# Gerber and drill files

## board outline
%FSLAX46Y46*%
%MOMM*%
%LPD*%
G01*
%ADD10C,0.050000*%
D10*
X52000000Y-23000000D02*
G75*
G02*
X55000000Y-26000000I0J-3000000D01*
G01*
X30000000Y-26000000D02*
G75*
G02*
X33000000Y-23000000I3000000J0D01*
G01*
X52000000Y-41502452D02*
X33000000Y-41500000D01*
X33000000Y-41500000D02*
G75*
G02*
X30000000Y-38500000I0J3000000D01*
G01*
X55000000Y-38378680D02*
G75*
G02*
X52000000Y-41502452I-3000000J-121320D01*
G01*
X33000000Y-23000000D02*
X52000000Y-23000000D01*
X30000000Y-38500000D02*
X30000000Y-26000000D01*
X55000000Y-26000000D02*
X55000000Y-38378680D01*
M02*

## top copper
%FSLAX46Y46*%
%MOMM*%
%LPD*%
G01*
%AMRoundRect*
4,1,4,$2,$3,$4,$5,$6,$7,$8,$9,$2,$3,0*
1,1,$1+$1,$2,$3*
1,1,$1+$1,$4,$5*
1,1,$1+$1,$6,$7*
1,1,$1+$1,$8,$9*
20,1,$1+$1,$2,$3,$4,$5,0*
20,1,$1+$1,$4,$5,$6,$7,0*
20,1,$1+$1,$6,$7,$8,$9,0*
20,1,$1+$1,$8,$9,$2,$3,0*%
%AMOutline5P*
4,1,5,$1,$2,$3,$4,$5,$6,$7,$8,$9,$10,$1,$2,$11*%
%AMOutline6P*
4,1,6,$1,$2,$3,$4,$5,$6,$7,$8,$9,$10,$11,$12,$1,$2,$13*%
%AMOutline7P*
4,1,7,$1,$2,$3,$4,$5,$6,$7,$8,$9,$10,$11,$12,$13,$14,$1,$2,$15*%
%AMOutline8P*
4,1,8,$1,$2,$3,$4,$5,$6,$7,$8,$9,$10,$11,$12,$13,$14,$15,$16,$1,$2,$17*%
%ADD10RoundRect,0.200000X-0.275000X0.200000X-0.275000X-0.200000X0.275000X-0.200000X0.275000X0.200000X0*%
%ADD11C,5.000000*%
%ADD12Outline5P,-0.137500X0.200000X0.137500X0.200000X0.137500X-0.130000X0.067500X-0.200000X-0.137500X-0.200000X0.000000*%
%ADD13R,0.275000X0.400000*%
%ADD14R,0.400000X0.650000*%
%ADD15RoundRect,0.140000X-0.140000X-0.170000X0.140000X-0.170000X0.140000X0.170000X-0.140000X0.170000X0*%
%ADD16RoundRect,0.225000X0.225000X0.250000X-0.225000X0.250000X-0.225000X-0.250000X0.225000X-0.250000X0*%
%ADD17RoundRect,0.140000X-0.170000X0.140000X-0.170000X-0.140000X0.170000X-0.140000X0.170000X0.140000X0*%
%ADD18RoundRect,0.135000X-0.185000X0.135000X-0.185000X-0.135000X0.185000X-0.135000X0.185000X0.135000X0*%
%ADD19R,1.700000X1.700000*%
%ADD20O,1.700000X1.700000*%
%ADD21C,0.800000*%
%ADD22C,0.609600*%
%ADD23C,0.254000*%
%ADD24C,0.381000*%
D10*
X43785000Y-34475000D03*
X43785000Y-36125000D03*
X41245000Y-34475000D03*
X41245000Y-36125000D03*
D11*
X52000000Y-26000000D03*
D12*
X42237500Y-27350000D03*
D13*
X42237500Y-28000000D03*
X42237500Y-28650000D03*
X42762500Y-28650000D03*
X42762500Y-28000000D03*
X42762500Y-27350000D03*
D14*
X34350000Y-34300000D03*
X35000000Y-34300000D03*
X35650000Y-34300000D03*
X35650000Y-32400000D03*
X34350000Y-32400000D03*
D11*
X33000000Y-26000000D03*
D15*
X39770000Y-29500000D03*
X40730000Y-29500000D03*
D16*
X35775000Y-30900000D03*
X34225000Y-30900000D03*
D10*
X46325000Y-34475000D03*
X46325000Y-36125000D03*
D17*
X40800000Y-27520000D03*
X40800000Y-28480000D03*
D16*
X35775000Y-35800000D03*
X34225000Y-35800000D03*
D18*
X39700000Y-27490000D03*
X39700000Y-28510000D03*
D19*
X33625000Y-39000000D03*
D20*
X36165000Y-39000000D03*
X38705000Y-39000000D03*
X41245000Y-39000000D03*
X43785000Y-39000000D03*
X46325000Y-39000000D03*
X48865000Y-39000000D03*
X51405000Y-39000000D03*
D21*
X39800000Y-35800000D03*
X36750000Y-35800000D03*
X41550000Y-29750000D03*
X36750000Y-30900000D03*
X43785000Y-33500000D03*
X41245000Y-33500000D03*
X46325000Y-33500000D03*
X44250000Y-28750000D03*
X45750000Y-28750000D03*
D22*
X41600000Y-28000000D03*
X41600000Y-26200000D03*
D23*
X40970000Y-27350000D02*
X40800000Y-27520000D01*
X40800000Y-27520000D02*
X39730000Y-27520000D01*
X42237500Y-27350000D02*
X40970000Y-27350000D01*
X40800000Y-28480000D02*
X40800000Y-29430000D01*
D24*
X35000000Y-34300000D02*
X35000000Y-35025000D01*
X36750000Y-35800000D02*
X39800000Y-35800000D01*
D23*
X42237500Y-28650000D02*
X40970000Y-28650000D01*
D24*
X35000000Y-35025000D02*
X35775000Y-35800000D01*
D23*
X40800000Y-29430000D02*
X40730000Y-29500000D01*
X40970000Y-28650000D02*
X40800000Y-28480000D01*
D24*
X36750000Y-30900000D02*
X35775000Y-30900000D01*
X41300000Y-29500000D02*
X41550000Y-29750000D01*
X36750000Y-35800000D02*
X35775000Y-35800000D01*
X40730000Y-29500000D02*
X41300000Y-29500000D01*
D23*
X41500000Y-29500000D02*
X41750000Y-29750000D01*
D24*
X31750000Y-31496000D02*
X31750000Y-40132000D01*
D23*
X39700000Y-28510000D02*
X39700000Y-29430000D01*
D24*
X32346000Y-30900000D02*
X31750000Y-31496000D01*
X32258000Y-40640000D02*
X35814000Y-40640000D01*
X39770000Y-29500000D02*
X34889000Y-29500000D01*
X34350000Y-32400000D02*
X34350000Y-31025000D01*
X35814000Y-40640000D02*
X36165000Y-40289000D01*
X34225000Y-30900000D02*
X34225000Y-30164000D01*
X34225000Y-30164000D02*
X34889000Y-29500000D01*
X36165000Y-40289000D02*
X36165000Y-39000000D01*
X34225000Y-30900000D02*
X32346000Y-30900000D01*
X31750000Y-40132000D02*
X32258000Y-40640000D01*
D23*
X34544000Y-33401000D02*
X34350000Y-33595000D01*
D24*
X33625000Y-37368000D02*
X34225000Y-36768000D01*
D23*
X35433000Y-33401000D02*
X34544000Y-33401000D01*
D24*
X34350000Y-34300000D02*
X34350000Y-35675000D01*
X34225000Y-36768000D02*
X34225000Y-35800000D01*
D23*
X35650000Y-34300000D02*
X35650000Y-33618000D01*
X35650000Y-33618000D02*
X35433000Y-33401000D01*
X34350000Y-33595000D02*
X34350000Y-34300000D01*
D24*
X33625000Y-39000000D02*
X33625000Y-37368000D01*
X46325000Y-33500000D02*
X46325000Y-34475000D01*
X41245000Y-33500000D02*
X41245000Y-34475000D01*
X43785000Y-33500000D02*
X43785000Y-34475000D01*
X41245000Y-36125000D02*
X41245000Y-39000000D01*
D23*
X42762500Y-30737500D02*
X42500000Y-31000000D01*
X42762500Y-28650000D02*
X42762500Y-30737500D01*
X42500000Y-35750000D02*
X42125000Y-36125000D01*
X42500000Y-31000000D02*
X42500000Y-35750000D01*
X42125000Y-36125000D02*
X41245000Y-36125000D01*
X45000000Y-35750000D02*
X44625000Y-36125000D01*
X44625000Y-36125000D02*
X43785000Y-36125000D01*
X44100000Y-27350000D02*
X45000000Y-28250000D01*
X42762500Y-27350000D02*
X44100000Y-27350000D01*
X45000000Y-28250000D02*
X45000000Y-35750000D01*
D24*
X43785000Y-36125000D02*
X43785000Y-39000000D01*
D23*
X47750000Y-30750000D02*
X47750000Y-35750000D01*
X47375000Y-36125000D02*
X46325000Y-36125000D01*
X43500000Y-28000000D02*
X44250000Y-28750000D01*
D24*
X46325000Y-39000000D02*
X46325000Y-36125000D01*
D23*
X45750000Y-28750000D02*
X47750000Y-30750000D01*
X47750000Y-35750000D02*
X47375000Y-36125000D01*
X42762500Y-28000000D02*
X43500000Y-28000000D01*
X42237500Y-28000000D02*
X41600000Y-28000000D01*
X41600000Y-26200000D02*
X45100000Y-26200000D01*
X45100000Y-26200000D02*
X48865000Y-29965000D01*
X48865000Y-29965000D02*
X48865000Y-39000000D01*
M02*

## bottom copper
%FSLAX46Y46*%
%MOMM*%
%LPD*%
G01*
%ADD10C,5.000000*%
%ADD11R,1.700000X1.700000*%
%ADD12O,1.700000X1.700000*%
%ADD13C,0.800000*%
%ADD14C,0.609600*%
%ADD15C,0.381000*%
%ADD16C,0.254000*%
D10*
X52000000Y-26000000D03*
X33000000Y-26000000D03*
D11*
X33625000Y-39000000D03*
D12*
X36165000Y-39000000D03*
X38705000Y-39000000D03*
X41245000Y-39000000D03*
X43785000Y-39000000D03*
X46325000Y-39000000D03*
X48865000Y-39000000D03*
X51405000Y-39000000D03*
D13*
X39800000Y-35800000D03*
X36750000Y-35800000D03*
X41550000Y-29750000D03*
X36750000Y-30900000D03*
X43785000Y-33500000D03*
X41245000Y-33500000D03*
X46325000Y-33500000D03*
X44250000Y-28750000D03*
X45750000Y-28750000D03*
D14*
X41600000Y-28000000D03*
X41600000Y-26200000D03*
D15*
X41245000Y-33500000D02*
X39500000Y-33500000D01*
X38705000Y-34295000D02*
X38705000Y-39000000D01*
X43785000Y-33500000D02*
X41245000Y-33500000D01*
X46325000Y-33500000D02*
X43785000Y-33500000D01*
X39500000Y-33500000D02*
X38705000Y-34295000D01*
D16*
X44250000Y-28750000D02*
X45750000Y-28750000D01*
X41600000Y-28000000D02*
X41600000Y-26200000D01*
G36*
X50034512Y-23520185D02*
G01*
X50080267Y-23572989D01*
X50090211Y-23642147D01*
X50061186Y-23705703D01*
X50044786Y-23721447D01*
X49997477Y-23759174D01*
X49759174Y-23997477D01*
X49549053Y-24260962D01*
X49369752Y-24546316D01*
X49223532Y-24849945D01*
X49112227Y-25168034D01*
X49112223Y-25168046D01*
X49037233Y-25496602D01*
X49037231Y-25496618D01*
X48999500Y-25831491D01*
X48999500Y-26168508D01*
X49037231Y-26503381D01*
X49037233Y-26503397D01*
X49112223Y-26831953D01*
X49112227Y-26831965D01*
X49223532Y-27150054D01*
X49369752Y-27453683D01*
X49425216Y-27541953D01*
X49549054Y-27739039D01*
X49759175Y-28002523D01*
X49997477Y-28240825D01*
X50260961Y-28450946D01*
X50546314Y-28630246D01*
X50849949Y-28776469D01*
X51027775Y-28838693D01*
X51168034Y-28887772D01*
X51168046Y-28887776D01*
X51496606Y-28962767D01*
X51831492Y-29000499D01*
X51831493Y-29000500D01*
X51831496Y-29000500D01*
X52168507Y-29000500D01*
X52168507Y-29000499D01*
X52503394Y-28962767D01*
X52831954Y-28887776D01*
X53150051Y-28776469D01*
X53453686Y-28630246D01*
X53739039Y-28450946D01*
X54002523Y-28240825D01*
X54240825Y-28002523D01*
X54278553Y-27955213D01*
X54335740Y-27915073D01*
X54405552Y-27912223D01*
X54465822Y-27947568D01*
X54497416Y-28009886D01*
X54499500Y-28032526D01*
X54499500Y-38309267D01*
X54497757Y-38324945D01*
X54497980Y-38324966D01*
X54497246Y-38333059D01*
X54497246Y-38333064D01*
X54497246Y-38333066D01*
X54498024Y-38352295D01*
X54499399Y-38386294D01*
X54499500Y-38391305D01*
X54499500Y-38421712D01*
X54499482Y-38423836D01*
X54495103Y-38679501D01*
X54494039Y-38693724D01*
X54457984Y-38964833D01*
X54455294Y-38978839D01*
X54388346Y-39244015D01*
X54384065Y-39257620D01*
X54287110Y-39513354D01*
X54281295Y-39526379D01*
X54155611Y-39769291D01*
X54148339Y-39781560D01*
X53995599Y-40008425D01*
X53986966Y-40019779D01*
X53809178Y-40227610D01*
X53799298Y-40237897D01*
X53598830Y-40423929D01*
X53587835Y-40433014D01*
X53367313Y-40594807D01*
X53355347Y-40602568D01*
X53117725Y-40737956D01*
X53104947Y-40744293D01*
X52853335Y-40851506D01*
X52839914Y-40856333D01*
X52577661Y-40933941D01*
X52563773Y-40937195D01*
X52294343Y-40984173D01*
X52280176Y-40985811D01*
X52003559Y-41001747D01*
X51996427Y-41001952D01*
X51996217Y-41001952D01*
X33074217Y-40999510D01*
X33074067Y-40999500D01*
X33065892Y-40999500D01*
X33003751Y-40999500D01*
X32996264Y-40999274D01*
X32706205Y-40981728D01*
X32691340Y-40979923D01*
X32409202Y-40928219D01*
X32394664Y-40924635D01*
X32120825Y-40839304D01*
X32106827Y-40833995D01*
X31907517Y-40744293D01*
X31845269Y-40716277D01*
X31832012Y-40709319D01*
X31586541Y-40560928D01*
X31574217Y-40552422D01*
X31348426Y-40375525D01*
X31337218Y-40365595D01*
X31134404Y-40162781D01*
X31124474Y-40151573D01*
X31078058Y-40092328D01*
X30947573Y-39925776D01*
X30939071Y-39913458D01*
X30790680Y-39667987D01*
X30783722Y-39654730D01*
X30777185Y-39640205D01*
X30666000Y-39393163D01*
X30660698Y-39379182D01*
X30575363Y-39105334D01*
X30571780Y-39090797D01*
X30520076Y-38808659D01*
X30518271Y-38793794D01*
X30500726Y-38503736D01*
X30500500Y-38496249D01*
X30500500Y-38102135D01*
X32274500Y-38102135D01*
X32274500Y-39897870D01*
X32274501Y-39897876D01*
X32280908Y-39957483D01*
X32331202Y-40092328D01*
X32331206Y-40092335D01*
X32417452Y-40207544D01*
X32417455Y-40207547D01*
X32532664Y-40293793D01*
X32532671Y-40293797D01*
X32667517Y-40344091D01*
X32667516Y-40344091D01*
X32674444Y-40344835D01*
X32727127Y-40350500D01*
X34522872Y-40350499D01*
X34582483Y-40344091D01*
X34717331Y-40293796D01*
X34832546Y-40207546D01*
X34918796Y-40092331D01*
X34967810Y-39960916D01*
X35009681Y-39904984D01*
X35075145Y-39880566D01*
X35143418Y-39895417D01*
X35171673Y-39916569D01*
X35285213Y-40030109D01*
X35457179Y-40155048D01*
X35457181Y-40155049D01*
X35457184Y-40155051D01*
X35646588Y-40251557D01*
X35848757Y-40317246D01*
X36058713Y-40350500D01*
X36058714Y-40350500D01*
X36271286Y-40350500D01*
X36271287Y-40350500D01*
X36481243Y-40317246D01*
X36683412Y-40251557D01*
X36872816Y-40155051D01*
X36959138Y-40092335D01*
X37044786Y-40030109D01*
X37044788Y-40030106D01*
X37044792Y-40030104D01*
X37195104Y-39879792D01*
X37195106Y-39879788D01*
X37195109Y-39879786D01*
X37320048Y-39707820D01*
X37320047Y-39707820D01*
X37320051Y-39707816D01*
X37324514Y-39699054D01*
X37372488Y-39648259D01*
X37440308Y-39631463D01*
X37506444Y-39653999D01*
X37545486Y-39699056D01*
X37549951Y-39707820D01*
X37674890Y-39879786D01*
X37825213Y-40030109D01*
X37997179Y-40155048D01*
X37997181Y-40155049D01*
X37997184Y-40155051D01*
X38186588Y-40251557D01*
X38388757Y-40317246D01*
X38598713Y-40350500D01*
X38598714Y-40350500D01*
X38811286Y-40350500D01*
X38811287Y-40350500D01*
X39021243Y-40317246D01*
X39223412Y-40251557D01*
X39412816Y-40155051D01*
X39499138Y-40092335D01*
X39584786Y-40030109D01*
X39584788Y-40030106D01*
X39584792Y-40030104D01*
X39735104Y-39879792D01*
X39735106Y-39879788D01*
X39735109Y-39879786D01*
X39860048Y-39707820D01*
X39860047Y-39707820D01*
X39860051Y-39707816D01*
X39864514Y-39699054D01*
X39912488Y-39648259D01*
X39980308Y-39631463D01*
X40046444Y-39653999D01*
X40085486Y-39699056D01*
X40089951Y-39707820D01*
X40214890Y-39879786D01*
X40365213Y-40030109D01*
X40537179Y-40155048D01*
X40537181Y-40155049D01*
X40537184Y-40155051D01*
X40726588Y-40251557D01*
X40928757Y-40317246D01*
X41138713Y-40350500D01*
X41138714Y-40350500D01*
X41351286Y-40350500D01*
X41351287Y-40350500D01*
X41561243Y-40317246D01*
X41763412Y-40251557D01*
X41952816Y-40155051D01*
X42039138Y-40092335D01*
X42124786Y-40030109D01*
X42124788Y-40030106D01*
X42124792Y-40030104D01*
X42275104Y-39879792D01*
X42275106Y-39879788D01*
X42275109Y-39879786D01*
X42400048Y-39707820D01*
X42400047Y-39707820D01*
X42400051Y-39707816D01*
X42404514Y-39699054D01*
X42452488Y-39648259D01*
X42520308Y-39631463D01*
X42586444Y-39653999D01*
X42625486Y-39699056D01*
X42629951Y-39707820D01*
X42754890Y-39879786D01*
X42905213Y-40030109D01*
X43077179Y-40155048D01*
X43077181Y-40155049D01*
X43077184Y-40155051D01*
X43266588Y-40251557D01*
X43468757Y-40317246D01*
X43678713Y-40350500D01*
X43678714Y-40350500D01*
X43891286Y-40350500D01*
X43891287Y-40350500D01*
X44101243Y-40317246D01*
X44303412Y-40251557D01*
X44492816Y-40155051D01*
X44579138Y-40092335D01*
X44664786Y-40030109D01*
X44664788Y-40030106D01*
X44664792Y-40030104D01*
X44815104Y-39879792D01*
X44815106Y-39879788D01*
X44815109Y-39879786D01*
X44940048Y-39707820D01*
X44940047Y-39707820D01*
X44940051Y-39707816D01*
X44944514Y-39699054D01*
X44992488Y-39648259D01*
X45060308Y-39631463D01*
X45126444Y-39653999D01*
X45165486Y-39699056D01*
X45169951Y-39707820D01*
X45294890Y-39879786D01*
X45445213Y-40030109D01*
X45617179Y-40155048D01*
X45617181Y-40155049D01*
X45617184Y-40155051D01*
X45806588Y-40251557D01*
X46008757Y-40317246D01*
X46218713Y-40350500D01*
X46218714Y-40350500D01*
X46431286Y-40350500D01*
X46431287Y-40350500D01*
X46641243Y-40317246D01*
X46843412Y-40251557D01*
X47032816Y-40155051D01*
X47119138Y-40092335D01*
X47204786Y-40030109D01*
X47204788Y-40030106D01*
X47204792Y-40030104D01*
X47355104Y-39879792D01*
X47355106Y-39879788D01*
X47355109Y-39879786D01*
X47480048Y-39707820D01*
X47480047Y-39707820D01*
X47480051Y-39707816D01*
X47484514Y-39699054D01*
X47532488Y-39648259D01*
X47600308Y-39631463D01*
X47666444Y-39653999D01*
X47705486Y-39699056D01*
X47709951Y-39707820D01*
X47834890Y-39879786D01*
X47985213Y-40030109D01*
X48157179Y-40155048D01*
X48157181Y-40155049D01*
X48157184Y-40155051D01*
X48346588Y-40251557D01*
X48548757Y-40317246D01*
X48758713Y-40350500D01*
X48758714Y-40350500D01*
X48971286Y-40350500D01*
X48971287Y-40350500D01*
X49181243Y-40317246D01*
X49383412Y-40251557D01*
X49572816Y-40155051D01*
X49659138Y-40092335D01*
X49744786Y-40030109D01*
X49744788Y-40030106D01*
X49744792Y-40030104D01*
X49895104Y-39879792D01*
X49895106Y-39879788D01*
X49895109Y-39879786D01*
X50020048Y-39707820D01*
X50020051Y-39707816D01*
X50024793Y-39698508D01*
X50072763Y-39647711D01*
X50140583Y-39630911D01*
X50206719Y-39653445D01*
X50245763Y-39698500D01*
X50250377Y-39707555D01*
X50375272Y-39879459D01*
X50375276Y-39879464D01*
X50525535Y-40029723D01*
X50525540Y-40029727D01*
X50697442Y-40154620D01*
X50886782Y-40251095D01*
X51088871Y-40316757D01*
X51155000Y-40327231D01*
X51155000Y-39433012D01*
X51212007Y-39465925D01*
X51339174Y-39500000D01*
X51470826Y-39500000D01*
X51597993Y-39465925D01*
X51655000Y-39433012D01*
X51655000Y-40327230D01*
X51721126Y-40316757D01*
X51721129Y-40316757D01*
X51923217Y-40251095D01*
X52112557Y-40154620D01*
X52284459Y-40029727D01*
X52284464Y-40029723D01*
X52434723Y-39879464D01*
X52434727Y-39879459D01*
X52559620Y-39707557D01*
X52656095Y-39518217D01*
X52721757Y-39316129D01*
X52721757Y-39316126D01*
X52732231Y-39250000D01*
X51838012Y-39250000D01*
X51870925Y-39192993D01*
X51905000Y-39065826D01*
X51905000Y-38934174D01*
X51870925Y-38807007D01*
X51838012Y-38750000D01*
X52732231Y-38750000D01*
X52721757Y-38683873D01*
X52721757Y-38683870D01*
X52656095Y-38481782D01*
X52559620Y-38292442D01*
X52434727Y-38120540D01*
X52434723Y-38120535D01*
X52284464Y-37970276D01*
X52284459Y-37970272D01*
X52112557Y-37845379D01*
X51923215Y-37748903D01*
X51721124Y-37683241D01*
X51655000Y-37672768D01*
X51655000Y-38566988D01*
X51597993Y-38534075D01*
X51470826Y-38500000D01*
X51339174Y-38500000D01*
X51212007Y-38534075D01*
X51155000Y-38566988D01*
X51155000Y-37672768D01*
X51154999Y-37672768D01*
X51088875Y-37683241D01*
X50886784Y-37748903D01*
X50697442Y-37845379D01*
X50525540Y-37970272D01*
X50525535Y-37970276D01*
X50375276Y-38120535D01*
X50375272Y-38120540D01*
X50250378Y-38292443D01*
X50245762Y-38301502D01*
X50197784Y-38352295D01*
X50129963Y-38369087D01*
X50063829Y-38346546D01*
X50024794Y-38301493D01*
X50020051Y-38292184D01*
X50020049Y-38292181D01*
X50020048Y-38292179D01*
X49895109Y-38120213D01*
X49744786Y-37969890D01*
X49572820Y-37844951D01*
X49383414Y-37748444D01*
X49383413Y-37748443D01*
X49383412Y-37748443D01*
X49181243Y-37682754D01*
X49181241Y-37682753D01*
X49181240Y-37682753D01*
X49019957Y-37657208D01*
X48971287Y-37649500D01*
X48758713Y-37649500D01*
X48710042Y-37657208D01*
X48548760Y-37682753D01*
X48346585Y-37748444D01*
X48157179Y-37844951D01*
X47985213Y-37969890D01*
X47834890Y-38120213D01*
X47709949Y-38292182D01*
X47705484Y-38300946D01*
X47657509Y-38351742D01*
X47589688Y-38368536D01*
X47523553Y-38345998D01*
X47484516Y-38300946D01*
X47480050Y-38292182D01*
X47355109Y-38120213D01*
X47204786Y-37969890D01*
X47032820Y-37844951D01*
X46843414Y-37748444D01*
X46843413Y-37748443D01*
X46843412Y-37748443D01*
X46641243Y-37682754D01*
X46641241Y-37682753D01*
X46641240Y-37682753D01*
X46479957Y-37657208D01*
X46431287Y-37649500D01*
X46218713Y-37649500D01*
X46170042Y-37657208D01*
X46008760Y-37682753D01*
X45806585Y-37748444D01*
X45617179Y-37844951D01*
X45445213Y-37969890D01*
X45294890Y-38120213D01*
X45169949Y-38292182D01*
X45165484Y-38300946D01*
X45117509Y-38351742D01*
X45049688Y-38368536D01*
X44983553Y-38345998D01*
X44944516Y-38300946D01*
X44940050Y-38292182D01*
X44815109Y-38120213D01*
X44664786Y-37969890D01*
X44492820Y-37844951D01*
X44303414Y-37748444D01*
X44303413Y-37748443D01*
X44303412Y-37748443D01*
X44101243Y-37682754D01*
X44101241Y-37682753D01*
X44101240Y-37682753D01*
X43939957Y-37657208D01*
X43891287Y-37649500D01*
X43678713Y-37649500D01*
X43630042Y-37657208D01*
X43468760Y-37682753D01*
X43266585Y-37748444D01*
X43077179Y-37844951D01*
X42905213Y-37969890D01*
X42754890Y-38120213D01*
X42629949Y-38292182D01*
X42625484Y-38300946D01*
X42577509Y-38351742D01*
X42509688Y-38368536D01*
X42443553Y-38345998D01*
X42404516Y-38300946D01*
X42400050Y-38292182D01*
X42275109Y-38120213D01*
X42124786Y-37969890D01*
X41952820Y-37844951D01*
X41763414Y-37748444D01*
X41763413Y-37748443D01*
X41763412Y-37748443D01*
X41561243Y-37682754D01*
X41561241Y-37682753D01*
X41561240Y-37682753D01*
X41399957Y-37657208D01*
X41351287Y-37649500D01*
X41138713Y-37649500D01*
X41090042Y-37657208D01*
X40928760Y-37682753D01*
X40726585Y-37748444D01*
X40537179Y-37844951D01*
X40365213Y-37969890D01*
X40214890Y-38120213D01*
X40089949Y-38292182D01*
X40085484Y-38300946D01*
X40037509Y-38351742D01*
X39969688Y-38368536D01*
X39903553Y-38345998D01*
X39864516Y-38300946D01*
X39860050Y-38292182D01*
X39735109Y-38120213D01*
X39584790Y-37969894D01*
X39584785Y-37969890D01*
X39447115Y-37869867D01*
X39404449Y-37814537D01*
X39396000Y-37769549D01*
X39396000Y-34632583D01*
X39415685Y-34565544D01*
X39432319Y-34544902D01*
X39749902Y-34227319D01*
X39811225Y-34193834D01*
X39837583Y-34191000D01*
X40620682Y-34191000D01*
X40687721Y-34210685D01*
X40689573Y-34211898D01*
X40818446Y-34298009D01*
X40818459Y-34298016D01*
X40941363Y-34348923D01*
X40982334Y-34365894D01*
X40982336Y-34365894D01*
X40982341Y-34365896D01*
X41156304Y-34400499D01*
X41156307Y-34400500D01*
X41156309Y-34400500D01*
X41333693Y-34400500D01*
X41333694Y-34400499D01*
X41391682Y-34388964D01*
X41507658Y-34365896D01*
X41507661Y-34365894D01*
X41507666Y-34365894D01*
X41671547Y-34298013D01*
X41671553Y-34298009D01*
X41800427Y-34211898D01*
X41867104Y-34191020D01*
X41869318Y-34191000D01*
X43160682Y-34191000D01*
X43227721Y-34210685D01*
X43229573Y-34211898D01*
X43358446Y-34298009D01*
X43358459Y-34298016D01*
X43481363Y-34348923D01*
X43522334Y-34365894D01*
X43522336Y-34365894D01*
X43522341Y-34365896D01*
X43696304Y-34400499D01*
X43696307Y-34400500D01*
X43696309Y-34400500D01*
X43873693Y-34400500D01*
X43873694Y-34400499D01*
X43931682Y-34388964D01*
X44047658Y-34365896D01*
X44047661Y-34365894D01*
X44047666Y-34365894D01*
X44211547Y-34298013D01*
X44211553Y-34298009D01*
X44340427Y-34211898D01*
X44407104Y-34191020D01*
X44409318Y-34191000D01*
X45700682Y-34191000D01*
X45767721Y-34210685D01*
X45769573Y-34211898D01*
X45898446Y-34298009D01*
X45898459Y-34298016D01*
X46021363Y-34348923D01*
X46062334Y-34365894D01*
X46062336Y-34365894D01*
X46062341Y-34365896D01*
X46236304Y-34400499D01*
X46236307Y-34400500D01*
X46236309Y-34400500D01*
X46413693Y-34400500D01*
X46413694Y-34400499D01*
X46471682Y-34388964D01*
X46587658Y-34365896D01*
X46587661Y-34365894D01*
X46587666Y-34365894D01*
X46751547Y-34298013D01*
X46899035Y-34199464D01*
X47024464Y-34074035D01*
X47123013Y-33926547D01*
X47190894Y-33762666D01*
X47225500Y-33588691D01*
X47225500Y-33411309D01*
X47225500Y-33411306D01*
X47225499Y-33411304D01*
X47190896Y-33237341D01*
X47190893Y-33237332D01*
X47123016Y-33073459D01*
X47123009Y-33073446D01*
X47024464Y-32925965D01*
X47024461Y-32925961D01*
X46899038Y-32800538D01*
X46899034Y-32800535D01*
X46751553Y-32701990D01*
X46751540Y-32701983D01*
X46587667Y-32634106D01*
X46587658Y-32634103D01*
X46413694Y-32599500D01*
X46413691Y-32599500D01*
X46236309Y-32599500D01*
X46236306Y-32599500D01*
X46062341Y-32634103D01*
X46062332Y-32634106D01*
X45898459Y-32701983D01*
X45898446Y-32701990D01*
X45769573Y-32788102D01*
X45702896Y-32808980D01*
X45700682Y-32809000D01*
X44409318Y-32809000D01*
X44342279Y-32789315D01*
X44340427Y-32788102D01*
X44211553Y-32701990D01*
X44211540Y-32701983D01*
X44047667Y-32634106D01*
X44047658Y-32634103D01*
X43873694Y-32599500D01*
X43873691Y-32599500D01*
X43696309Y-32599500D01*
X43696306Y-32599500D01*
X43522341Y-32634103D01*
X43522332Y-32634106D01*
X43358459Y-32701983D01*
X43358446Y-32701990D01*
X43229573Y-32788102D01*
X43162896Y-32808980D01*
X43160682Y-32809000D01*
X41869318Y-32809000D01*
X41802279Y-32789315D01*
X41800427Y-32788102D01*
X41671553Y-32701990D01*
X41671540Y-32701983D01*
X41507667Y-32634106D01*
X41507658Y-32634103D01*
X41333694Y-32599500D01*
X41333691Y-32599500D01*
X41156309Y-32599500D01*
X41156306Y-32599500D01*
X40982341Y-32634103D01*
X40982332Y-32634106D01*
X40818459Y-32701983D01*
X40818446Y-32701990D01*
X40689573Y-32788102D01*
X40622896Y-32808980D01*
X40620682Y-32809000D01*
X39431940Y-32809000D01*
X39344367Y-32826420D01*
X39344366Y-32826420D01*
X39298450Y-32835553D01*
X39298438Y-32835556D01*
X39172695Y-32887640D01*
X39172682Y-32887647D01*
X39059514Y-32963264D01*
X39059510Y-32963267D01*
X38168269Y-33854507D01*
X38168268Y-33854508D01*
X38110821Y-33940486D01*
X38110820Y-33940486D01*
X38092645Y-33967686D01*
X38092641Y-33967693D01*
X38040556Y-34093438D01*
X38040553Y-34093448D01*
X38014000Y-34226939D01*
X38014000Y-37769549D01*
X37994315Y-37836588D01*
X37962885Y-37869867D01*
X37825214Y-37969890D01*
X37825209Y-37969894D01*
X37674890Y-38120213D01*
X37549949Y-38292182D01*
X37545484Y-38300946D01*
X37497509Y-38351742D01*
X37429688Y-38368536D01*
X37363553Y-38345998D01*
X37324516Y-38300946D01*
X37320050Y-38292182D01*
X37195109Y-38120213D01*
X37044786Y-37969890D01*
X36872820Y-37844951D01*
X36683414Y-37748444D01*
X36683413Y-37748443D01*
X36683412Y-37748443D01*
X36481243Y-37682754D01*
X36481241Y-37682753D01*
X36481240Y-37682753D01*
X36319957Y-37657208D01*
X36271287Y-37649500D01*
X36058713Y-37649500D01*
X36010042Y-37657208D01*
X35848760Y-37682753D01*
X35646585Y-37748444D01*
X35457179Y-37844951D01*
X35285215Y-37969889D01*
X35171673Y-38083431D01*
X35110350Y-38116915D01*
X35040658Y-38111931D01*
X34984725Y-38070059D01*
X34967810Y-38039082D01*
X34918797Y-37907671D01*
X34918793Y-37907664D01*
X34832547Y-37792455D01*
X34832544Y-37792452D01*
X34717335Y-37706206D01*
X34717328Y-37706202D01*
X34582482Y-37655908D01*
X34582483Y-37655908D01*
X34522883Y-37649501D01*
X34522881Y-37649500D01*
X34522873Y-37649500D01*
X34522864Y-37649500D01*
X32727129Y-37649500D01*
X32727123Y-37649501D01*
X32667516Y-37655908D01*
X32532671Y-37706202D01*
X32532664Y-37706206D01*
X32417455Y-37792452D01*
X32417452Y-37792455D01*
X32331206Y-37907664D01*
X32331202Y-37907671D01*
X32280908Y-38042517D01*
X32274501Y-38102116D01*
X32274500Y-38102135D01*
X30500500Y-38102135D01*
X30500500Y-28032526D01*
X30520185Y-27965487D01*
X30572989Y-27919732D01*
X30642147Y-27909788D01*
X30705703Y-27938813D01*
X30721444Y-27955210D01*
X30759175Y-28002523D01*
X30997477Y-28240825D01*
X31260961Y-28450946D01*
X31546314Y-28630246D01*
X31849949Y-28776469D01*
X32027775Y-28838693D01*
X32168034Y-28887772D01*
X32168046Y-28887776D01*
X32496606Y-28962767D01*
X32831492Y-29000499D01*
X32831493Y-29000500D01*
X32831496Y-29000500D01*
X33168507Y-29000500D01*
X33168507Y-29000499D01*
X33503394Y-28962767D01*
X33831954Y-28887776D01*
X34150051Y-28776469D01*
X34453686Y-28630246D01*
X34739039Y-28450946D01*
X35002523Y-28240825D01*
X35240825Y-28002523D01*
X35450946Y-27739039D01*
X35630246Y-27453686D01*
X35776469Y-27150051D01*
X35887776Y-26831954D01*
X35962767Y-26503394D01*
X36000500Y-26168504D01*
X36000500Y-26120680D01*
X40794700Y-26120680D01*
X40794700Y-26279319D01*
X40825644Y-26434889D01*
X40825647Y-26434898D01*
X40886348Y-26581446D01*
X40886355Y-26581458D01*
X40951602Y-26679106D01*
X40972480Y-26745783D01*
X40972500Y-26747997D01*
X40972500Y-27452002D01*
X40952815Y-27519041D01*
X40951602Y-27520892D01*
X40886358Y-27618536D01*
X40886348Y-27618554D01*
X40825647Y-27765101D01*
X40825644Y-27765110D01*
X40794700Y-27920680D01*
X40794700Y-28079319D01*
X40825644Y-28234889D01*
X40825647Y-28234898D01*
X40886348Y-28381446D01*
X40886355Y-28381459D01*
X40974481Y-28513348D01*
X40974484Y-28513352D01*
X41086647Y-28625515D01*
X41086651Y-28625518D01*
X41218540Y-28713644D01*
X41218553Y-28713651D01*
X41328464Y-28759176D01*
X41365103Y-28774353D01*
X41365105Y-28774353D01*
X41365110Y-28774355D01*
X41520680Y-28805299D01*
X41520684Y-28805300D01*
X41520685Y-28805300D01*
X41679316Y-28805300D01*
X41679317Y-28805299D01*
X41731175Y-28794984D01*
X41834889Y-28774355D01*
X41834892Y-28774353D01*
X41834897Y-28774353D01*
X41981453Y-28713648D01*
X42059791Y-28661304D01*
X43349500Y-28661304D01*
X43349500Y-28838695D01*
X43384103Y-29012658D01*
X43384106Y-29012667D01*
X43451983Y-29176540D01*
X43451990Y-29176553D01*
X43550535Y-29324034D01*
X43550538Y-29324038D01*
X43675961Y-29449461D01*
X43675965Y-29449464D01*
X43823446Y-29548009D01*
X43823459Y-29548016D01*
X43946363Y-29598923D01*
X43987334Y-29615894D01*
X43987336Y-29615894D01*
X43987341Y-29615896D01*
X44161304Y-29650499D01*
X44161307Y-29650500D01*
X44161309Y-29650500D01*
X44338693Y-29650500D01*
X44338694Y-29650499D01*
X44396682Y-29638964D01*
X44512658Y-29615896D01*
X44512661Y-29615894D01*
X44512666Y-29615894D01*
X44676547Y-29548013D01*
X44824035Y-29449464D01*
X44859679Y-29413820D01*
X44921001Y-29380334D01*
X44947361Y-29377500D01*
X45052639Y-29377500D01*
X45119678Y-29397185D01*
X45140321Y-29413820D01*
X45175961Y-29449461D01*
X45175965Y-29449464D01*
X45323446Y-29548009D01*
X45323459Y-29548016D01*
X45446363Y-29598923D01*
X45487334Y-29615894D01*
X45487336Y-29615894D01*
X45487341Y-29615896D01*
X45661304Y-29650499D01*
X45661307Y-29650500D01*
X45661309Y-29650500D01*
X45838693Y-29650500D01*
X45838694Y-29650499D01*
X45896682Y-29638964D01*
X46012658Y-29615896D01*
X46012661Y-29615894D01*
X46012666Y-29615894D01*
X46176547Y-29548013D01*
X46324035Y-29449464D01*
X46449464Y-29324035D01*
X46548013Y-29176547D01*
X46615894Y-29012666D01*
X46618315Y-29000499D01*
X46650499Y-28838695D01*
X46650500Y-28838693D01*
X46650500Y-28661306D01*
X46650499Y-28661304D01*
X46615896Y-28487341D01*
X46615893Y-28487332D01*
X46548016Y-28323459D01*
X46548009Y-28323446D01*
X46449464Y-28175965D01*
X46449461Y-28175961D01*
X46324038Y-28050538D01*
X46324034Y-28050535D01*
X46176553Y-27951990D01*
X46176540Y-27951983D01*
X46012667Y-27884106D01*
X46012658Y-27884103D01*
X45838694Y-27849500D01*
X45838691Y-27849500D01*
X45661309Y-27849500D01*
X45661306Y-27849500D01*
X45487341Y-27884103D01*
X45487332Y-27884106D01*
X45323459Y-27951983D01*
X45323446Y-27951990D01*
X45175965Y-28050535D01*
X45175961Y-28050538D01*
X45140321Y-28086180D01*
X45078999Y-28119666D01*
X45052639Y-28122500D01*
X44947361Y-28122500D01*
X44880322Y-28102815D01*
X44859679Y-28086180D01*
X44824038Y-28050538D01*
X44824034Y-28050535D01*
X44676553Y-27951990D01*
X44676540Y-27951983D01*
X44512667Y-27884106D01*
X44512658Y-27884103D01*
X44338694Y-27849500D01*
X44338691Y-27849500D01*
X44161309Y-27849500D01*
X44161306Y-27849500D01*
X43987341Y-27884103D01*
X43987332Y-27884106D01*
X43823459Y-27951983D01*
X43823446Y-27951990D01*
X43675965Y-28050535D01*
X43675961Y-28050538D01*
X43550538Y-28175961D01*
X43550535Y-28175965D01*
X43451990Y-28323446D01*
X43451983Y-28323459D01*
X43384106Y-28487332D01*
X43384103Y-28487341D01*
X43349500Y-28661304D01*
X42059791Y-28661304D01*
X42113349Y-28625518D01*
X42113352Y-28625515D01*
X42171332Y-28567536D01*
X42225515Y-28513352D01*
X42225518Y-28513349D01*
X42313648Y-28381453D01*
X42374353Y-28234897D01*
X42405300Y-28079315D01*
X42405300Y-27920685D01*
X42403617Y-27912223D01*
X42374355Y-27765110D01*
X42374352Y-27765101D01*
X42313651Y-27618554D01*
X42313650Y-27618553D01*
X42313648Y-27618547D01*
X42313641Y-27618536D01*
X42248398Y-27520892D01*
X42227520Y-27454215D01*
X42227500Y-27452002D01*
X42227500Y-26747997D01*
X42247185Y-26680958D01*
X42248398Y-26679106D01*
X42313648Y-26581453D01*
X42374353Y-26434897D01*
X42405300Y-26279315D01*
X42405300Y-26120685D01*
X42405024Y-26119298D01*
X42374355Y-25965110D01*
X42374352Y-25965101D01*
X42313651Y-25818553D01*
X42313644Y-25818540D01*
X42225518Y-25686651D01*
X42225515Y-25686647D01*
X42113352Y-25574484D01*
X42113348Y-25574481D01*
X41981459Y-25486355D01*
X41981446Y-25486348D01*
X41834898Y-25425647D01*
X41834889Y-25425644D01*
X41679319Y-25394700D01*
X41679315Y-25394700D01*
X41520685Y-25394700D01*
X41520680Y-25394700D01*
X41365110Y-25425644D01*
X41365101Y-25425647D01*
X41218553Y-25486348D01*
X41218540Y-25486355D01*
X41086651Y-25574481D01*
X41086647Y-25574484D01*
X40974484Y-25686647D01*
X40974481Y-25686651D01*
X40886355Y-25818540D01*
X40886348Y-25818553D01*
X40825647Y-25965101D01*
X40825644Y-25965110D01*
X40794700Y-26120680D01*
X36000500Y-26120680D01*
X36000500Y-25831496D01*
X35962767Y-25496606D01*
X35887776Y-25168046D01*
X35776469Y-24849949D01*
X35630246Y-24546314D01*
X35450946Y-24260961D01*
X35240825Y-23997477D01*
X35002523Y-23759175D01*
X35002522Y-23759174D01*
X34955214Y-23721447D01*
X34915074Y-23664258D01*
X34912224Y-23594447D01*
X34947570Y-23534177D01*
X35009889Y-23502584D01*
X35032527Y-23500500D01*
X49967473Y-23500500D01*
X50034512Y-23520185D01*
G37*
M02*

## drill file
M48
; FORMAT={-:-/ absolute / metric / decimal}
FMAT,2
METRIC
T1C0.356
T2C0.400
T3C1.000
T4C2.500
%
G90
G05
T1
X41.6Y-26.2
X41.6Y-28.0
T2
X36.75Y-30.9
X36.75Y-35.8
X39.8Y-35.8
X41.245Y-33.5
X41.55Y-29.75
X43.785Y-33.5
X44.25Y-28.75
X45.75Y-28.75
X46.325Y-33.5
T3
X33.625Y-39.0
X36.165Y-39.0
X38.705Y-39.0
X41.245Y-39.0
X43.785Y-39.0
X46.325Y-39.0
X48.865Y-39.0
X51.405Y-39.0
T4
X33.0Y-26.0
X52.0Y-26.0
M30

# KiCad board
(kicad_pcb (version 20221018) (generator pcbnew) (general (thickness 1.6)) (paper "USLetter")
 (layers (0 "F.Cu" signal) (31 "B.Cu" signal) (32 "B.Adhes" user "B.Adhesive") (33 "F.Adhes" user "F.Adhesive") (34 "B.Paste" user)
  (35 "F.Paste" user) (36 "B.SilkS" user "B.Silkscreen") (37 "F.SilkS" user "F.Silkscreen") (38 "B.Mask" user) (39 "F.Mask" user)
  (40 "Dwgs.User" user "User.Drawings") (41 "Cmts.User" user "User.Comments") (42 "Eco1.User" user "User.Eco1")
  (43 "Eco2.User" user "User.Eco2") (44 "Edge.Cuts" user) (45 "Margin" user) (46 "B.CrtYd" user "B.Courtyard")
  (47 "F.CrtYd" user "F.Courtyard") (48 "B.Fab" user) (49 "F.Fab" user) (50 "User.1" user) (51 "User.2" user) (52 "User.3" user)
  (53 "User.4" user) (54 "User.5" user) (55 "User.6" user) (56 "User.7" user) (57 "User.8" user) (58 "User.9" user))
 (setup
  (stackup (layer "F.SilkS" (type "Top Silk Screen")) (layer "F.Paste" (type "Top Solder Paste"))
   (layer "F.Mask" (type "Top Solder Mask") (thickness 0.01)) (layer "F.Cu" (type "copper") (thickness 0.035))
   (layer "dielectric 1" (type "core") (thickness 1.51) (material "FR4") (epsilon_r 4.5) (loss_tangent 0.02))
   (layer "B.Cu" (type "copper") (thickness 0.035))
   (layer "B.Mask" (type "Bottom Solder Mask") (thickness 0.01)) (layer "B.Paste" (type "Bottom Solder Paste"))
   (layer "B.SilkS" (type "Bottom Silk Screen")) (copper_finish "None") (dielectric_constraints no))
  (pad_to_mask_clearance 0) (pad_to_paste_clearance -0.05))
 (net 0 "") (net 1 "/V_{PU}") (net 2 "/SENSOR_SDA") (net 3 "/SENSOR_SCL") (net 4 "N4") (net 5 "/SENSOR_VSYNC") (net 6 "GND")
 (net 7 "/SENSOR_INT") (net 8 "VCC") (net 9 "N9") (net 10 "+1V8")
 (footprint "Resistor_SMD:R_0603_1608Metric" (layer "F.Cu") (at 43.785 35.3 -90)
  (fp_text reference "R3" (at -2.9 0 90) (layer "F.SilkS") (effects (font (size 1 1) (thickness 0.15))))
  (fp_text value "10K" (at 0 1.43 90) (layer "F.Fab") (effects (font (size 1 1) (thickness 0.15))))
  (pad "1" smd roundrect (at -0.825 0 270) (size 0.8 0.95) (layers "F.Cu" "F.Paste" "F.Mask") (roundrect_rratio 0.25) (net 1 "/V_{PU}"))
  (pad "2" smd roundrect (at 0.825 0 270) (size 0.8 0.95) (layers "F.Cu" "F.Paste" "F.Mask") (roundrect_rratio 0.25) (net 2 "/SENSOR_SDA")))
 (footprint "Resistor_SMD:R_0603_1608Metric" (layer "F.Cu") (at 41.245 35.3 -90)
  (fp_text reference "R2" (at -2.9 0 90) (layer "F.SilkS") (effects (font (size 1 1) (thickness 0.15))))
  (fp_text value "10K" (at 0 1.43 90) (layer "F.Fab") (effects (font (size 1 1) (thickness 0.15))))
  (pad "1" smd roundrect (at -0.825 0 270) (size 0.8 0.95) (layers "F.Cu" "F.Paste" "F.Mask") (roundrect_rratio 0.25) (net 1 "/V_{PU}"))
  (pad "2" smd roundrect (at 0.825 0 270) (size 0.8 0.95) (layers "F.Cu" "F.Paste" "F.Mask") (roundrect_rratio 0.25) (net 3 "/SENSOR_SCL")))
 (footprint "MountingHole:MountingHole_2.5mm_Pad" (layer "F.Cu") (at 52 26)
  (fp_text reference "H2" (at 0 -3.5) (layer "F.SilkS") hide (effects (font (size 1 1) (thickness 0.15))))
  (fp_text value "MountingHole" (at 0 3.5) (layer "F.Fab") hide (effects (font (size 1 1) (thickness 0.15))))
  (pad "1" thru_hole circle (at 0 0) (size 5 5) (drill 2.5) (layers "*.Cu" "*.Mask")))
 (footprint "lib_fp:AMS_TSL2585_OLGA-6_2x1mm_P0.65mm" (layer "F.Cu") (at 42.5 28) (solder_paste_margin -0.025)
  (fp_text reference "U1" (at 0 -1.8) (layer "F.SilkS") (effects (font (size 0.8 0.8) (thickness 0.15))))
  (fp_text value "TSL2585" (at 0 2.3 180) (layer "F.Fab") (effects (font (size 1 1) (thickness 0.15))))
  (pad "1" smd roundrect (at -0.2625 -0.65) (size 0.275 0.4) (layers "F.Cu" "F.Paste" "F.Mask") (roundrect_rratio 0)
   (chamfer_ratio 0.254545) (chamfer bottom_right) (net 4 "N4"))
  (pad "2" smd rect (at -0.2625 0) (size 0.275 0.4) (layers "F.Cu" "F.Paste" "F.Mask") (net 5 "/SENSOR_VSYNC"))
  (pad "3" smd rect (at -0.2625 0.65) (size 0.275 0.4) (layers "F.Cu" "F.Paste" "F.Mask") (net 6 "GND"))
  (pad "4" smd rect (at 0.2625 0.65) (size 0.275 0.4) (layers "F.Cu" "F.Paste" "F.Mask") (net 3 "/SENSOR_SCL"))
  (pad "5" smd rect (at 0.2625 0) (size 0.275 0.4) (layers "F.Cu" "F.Paste" "F.Mask") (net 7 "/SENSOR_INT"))
  (pad "6" smd rect (at 0.2625 -0.65) (size 0.275 0.4) (layers "F.Cu" "F.Paste" "F.Mask") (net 2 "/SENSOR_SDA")))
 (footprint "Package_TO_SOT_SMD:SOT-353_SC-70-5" (layer "F.Cu") (at 35 33.35 90)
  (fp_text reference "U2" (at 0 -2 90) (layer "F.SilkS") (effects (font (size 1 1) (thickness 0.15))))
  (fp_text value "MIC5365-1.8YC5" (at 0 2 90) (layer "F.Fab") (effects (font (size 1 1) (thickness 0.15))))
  (pad "1" smd rect (at -0.95 -0.65 90) (size 0.65 0.4) (layers "F.Cu" "F.Paste" "F.Mask") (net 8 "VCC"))
  (pad "2" smd rect (at -0.95 0 90) (size 0.65 0.4) (layers "F.Cu" "F.Paste" "F.Mask") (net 6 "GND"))
  (pad "3" smd rect (at -0.95 0.65 90) (size 0.65 0.4) (layers "F.Cu" "F.Paste" "F.Mask") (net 8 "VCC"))
  (pad "4" smd rect (at 0.95 0.65 90) (size 0.65 0.4) (layers "F.Cu" "F.Paste" "F.Mask") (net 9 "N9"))
  (pad "5" smd rect (at 0.95 -0.65 90) (size 0.65 0.4) (layers "F.Cu" "F.Paste" "F.Mask") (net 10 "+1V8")))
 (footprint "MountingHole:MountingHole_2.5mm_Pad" (layer "F.Cu") (at 33 26)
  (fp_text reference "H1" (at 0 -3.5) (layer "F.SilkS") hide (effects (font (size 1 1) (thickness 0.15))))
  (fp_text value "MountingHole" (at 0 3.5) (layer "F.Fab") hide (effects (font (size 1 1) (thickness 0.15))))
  (pad "1" thru_hole circle (at 0 0) (size 5 5) (drill 2.5) (layers "*.Cu" "*.Mask")))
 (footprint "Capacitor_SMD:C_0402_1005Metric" (layer "F.Cu") (at 40.25 29.5)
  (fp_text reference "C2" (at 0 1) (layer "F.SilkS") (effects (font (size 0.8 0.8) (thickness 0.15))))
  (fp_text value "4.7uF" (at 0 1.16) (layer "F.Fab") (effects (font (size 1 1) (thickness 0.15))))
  (pad "1" smd roundrect (at -0.48 0) (size 0.56 0.62) (layers "F.Cu" "F.Paste" "F.Mask") (roundrect_rratio 0.25) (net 10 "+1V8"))
  (pad "2" smd roundrect (at 0.48 0) (size 0.56 0.62) (layers "F.Cu" "F.Paste" "F.Mask") (roundrect_rratio 0.25) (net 6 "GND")))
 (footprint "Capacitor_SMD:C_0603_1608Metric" (layer "F.Cu") (at 35 30.9 180)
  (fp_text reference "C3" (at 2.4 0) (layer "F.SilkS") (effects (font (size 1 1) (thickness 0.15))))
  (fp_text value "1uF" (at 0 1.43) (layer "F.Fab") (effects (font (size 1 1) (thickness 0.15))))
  (pad "1" smd roundrect (at -0.775 0 180) (size 0.9 0.95) (layers "F.Cu" "F.Paste" "F.Mask") (roundrect_rratio 0.25) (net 6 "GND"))
  (pad "2" smd roundrect (at 0.775 0 180) (size 0.9 0.95) (layers "F.Cu" "F.Paste" "F.Mask") (roundrect_rratio 0.25) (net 10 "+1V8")))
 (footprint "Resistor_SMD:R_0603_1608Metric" (layer "F.Cu") (at 46.325 35.3 -90)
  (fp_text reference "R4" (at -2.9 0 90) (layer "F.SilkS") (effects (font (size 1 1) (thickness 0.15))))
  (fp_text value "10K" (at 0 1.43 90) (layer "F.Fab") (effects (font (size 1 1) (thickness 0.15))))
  (pad "1" smd roundrect (at -0.825 0 270) (size 0.8 0.95) (layers "F.Cu" "F.Paste" "F.Mask") (roundrect_rratio 0.25) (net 1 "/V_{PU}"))
  (pad "2" smd roundrect (at 0.825 0 270) (size 0.8 0.95) (layers "F.Cu" "F.Paste" "F.Mask") (roundrect_rratio 0.25) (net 7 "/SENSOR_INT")))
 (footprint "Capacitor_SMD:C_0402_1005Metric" (layer "F.Cu") (at 40.8 28 -90)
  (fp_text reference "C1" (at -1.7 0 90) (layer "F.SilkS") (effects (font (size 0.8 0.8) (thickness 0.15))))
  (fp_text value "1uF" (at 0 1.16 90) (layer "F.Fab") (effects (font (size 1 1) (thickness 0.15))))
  (pad "1" smd roundrect (at -0.48 0 270) (size 0.56 0.62) (layers "F.Cu" "F.Paste" "F.Mask") (roundrect_rratio 0.25) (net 4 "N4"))
  (pad "2" smd roundrect (at 0.48 0 270) (size 0.56 0.62) (layers "F.Cu" "F.Paste" "F.Mask") (roundrect_rratio 0.25) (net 6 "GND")))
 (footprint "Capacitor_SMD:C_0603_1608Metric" (layer "F.Cu") (at 35 35.8 180)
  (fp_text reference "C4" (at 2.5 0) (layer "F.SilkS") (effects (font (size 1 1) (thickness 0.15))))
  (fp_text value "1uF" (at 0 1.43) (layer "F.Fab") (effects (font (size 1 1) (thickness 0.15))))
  (pad "1" smd roundrect (at -0.775 0 180) (size 0.9 0.95) (layers "F.Cu" "F.Paste" "F.Mask") (roundrect_rratio 0.25) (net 6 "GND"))
  (pad "2" smd roundrect (at 0.775 0 180) (size 0.9 0.95) (layers "F.Cu" "F.Paste" "F.Mask") (roundrect_rratio 0.25) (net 8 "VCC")))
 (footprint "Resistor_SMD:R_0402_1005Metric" (layer "F.Cu") (at 39.7 28 -90)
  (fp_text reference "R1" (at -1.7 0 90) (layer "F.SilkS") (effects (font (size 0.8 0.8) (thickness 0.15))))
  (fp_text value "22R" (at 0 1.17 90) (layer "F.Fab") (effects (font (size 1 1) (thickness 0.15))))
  (pad "1" smd roundrect (at -0.51 0 270) (size 0.54 0.64) (layers "F.Cu" "F.Paste" "F.Mask") (roundrect_rratio 0.25) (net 4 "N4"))
  (pad "2" smd roundrect (at 0.51 0 270) (size 0.54 0.64) (layers "F.Cu" "F.Paste" "F.Mask") (roundrect_rratio 0.25) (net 10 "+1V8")))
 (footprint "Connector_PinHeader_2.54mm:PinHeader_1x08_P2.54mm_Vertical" (layer "B.Cu") (at 33.625 39 -90)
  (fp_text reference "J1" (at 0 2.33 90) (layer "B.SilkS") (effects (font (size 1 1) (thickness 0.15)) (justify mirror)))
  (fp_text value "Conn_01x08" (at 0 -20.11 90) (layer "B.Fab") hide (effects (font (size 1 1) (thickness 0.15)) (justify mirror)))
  (pad "1" thru_hole rect (at 0 0 270) (size 1.7 1.7) (drill 1) (layers "*.Cu" "*.Mask") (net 8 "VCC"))
  (pad "2" thru_hole oval (at 0 -2.54 270) (size 1.7 1.7) (drill 1) (layers "*.Cu" "*.Mask") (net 10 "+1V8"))
  (pad "3" thru_hole oval (at 0 -5.08 270) (size 1.7 1.7) (drill 1) (layers "*.Cu" "*.Mask") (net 1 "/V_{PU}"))
  (pad "4" thru_hole oval (at 0 -7.62 270) (size 1.7 1.7) (drill 1) (layers "*.Cu" "*.Mask") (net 3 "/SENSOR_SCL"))
  (pad "5" thru_hole oval (at 0 -10.16 270) (size 1.7 1.7) (drill 1) (layers "*.Cu" "*.Mask") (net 2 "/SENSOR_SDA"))
  (pad "6" thru_hole oval (at 0 -12.7 270) (size 1.7 1.7) (drill 1) (layers "*.Cu" "*.Mask") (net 7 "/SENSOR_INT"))
  (pad "7" thru_hole oval (at 0 -15.24 270) (size 1.7 1.7) (drill 1) (layers "*.Cu" "*.Mask") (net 5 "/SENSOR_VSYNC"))
  (pad "8" thru_hole oval (at 0 -17.78 270) (size 1.7 1.7) (drill 1) (layers "*.Cu" "*.Mask") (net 6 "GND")))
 (gr_arc (start 52 23) (mid 54.12132 23.87868) (end 55 26) (stroke (width 0.05) (type default)) (layer "Edge.Cuts"))
 (gr_arc (start 30 26) (mid 30.87868 23.87868) (end 33 23) (stroke (width 0.05) (type default)) (layer "Edge.Cuts"))
 (gr_line (start 52 41.502452) (end 33 41.5) (stroke (width 0.05) (type default)) (layer "Edge.Cuts"))
 (gr_arc (start 33 41.5) (mid 30.87868 40.62132) (end 30 38.5) (stroke (width 0.05) (type default)) (layer "Edge.Cuts"))
 (gr_arc (start 55 38.37868) (mid 54.165523 40.579719) (end 52 41.502452) (stroke (width 0.05) (type default)) (layer "Edge.Cuts"))
 (gr_line (start 33 23) (end 52 23) (stroke (width 0.05) (type default)) (layer "Edge.Cuts"))
 (gr_line (start 30 38.5) (end 30 26) (stroke (width 0.05) (type default)) (layer "Edge.Cuts"))
 (gr_line (start 55 26) (end 55 38.37868) (stroke (width 0.05) (type default)) (layer "Edge.Cuts"))
 (segment (start 40.97 27.35) (end 40.8 27.52) (width 0.254) (layer "F.Cu") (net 4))
 (segment (start 40.8 27.52) (end 39.73 27.52) (width 0.254) (layer "F.Cu") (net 4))
 (segment (start 42.2375 27.35) (end 40.97 27.35) (width 0.254) (layer "F.Cu") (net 4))
 (segment (start 40.8 28.48) (end 40.8 29.43) (width 0.254) (layer "F.Cu") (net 6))
 (segment (start 35 34.3) (end 35 35.025) (width 0.381) (layer "F.Cu") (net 6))
 (segment (start 36.75 35.8) (end 39.8 35.8) (width 0.381) (layer "F.Cu") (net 6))
 (segment (start 42.2375 28.65) (end 40.97 28.65) (width 0.254) (layer "F.Cu") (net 6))
 (segment (start 35 35.025) (end 35.775 35.8) (width 0.381) (layer "F.Cu") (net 6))
 (segment (start 40.8 29.43) (end 40.73 29.5) (width 0.254) (layer "F.Cu") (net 6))
 (segment (start 40.97 28.65) (end 40.8 28.48) (width 0.254) (layer "F.Cu") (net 6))
 (segment (start 36.75 30.9) (end 35.775 30.9) (width 0.381) (layer "F.Cu") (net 6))
 (segment (start 41.3 29.5) (end 41.55 29.75) (width 0.381) (layer "F.Cu") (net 6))
 (segment (start 36.75 35.8) (end 35.775 35.8) (width 0.381) (layer "F.Cu") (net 6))
 (segment (start 40.73 29.5) (end 41.3 29.5) (width 0.381) (layer "F.Cu") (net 6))
 (segment (start 41.5 29.5) (end 41.75 29.75) (width 0.254) (layer "F.Cu") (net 6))
 (via (at 39.8 35.8) (size 0.8) (drill 0.4) (layers "F.Cu" "B.Cu") (free) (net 6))
 (via (at 36.75 35.8) (size 0.8) (drill 0.4) (layers "F.Cu" "B.Cu") (free) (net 6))
 (via (at 41.55 29.75) (size 0.8) (drill 0.4) (layers "F.Cu" "B.Cu") (free) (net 6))
 (via (at 36.75 30.9) (size 0.8) (drill 0.4) (layers "F.Cu" "B.Cu") (free) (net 6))
 (segment (start 31.75 31.496) (end 31.75 40.132) (width 0.381) (layer "F.Cu") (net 10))
 (segment (start 39.7 28.51) (end 39.7 29.43) (width 0.254) (layer "F.Cu") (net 10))
 (segment (start 32.346 30.9) (end 31.75 31.496) (width 0.381) (layer "F.Cu") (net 10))
 (segment (start 32.258 40.64) (end 35.814 40.64) (width 0.381) (layer "F.Cu") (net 10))
 (segment (start 39.77 29.5) (end 34.889 29.5) (width 0.381) (layer "F.Cu") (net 10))
 (segment (start 34.35 32.4) (end 34.35 31.025) (width 0.381) (layer "F.Cu") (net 10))
 (segment (start 35.814 40.64) (end 36.165 40.289) (width 0.381) (layer "F.Cu") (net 10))
 (segment (start 34.225 30.9) (end 34.225 30.164) (width 0.381) (layer "F.Cu") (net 10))
 (segment (start 34.225 30.164) (end 34.889 29.5) (width 0.381) (layer "F.Cu") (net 10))
 (segment (start 36.165 40.289) (end 36.165 39) (width 0.381) (layer "F.Cu") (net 10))
 (segment (start 34.225 30.9) (end 32.346 30.9) (width 0.381) (layer "F.Cu") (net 10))
 (segment (start 31.75 40.132) (end 32.258 40.64) (width 0.381) (layer "F.Cu") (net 10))
 (segment (start 34.544 33.401) (end 34.35 33.595) (width 0.254) (layer "F.Cu") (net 8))
 (segment (start 33.625 37.368) (end 34.225 36.768) (width 0.381) (layer "F.Cu") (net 8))
 (segment (start 35.433 33.401) (end 34.544 33.401) (width 0.254) (layer "F.Cu") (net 8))
 (segment (start 34.35 34.3) (end 34.35 35.675) (width 0.381) (layer "F.Cu") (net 8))
 (segment (start 34.225 36.768) (end 34.225 35.8) (width 0.381) (layer "F.Cu") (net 8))
 (segment (start 35.65 34.3) (end 35.65 33.618) (width 0.254) (layer "F.Cu") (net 8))
 (segment (start 35.65 33.618) (end 35.433 33.401) (width 0.254) (layer "F.Cu") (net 8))
 (segment (start 34.35 33.595) (end 34.35 34.3) (width 0.254) (layer "F.Cu") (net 8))
 (segment (start 33.625 39) (end 33.625 37.368) (width 0.381) (layer "F.Cu") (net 8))
 (segment (start 46.325 33.5) (end 46.325 34.475) (width 0.381) (layer "F.Cu") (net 1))
 (segment (start 41.245 33.5) (end 41.245 34.475) (width 0.381) (layer "F.Cu") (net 1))
 (segment (start 43.785 33.5) (end 43.785 34.475) (width 0.381) (layer "F.Cu") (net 1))
 (via (at 43.785 33.5) (size 0.8) (drill 0.4) (layers "F.Cu" "B.Cu") (free) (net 1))
 (via (at 41.245 33.5) (size 0.8) (drill 0.4) (layers "F.Cu" "B.Cu") (free) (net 1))
 (via (at 46.325 33.5) (size 0.8) (drill 0.4) (layers "F.Cu" "B.Cu") (free) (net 1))
 (segment (start 41.245 33.5) (end 39.5 33.5) (width 0.381) (layer "B.Cu") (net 1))
 (segment (start 38.705 34.295) (end 38.705 39) (width 0.381) (layer "B.Cu") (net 1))
 (segment (start 43.785 33.5) (end 41.245 33.5) (width 0.381) (layer "B.Cu") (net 1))
 (segment (start 46.325 33.5) (end 43.785 33.5) (width 0.381) (layer "B.Cu") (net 1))
 (segment (start 39.5 33.5) (end 38.705 34.295) (width 0.381) (layer "B.Cu") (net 1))
 (segment (start 41.245 36.125) (end 41.245 39) (width 0.381) (layer "F.Cu") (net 3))
 (segment (start 42.7625 30.7375) (end 42.5 31) (width 0.254) (layer "F.Cu") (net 3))
 (segment (start 42.7625 28.65) (end 42.7625 30.7375) (width 0.254) (layer "F.Cu") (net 3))
 (segment (start 42.5 35.75) (end 42.125 36.125) (width 0.254) (layer "F.Cu") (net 3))
 (segment (start 42.5 31) (end 42.5 35.75) (width 0.254) (layer "F.Cu") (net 3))
 (segment (start 42.125 36.125) (end 41.245 36.125) (width 0.254) (layer "F.Cu") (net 3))
 (segment (start 45 35.75) (end 44.625 36.125) (width 0.254) (layer "F.Cu") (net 2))
 (segment (start 44.625 36.125) (end 43.785 36.125) (width 0.254) (layer "F.Cu") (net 2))
 (segment (start 44.1 27.35) (end 45 28.25) (width 0.254) (layer "F.Cu") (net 2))
 (segment (start 42.7625 27.35) (end 44.1 27.35) (width 0.254) (layer "F.Cu") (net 2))
 (segment (start 45 28.25) (end 45 35.75) (width 0.254) (layer "F.Cu") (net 2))
 (segment (start 43.785 36.125) (end 43.785 39) (width 0.381) (layer "F.Cu") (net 2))
 (segment (start 47.75 30.75) (end 47.75 35.75) (width 0.254) (layer "F.Cu") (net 7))
 (segment (start 47.375 36.125) (end 46.325 36.125) (width 0.254) (layer "F.Cu") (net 7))
 (segment (start 43.5 28) (end 44.25 28.75) (width 0.254) (layer "F.Cu") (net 7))
 (segment (start 46.325 39) (end 46.325 36.125) (width 0.381) (layer "F.Cu") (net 7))
 (segment (start 45.75 28.75) (end 47.75 30.75) (width 0.254) (layer "F.Cu") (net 7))
 (segment (start 47.75 35.75) (end 47.375 36.125) (width 0.254) (layer "F.Cu") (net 7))
 (segment (start 42.7625 28) (end 43.5 28) (width 0.254) (layer "F.Cu") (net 7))
 (via (at 44.25 28.75) (size 0.8) (drill 0.4) (layers "F.Cu" "B.Cu") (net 7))
 (via (at 45.75 28.75) (size 0.8) (drill 0.4) (layers "F.Cu" "B.Cu") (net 7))
 (segment (start 44.25 28.75) (end 45.75 28.75) (width 0.254) (layer "B.Cu") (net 7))
 (segment (start 42.2375 28) (end 41.6 28) (width 0.254) (layer "F.Cu") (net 5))
 (segment (start 41.6 26.2) (end 45.1 26.2) (width 0.254) (layer "F.Cu") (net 5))
 (segment (start 45.1 26.2) (end 48.865 29.965) (width 0.254) (layer "F.Cu") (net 5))
 (segment (start 48.865 29.965) (end 48.865 39) (width 0.254) (layer "F.Cu") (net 5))
 (via (at 41.6 28) (size 0.6096) (drill 0.3556) (layers "F.Cu" "B.Cu") (free) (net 5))
 (via (at 41.6 26.2) (size 0.6096) (drill 0.3556) (layers "F.Cu" "B.Cu") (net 5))
 (segment (start 41.6 28) (end 41.6 26.2) (width 0.254) (layer "B.Cu") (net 5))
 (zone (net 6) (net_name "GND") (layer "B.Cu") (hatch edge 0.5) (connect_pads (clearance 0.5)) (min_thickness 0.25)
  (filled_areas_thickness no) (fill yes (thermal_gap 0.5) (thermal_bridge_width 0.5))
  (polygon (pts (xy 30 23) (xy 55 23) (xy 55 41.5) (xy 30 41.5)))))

